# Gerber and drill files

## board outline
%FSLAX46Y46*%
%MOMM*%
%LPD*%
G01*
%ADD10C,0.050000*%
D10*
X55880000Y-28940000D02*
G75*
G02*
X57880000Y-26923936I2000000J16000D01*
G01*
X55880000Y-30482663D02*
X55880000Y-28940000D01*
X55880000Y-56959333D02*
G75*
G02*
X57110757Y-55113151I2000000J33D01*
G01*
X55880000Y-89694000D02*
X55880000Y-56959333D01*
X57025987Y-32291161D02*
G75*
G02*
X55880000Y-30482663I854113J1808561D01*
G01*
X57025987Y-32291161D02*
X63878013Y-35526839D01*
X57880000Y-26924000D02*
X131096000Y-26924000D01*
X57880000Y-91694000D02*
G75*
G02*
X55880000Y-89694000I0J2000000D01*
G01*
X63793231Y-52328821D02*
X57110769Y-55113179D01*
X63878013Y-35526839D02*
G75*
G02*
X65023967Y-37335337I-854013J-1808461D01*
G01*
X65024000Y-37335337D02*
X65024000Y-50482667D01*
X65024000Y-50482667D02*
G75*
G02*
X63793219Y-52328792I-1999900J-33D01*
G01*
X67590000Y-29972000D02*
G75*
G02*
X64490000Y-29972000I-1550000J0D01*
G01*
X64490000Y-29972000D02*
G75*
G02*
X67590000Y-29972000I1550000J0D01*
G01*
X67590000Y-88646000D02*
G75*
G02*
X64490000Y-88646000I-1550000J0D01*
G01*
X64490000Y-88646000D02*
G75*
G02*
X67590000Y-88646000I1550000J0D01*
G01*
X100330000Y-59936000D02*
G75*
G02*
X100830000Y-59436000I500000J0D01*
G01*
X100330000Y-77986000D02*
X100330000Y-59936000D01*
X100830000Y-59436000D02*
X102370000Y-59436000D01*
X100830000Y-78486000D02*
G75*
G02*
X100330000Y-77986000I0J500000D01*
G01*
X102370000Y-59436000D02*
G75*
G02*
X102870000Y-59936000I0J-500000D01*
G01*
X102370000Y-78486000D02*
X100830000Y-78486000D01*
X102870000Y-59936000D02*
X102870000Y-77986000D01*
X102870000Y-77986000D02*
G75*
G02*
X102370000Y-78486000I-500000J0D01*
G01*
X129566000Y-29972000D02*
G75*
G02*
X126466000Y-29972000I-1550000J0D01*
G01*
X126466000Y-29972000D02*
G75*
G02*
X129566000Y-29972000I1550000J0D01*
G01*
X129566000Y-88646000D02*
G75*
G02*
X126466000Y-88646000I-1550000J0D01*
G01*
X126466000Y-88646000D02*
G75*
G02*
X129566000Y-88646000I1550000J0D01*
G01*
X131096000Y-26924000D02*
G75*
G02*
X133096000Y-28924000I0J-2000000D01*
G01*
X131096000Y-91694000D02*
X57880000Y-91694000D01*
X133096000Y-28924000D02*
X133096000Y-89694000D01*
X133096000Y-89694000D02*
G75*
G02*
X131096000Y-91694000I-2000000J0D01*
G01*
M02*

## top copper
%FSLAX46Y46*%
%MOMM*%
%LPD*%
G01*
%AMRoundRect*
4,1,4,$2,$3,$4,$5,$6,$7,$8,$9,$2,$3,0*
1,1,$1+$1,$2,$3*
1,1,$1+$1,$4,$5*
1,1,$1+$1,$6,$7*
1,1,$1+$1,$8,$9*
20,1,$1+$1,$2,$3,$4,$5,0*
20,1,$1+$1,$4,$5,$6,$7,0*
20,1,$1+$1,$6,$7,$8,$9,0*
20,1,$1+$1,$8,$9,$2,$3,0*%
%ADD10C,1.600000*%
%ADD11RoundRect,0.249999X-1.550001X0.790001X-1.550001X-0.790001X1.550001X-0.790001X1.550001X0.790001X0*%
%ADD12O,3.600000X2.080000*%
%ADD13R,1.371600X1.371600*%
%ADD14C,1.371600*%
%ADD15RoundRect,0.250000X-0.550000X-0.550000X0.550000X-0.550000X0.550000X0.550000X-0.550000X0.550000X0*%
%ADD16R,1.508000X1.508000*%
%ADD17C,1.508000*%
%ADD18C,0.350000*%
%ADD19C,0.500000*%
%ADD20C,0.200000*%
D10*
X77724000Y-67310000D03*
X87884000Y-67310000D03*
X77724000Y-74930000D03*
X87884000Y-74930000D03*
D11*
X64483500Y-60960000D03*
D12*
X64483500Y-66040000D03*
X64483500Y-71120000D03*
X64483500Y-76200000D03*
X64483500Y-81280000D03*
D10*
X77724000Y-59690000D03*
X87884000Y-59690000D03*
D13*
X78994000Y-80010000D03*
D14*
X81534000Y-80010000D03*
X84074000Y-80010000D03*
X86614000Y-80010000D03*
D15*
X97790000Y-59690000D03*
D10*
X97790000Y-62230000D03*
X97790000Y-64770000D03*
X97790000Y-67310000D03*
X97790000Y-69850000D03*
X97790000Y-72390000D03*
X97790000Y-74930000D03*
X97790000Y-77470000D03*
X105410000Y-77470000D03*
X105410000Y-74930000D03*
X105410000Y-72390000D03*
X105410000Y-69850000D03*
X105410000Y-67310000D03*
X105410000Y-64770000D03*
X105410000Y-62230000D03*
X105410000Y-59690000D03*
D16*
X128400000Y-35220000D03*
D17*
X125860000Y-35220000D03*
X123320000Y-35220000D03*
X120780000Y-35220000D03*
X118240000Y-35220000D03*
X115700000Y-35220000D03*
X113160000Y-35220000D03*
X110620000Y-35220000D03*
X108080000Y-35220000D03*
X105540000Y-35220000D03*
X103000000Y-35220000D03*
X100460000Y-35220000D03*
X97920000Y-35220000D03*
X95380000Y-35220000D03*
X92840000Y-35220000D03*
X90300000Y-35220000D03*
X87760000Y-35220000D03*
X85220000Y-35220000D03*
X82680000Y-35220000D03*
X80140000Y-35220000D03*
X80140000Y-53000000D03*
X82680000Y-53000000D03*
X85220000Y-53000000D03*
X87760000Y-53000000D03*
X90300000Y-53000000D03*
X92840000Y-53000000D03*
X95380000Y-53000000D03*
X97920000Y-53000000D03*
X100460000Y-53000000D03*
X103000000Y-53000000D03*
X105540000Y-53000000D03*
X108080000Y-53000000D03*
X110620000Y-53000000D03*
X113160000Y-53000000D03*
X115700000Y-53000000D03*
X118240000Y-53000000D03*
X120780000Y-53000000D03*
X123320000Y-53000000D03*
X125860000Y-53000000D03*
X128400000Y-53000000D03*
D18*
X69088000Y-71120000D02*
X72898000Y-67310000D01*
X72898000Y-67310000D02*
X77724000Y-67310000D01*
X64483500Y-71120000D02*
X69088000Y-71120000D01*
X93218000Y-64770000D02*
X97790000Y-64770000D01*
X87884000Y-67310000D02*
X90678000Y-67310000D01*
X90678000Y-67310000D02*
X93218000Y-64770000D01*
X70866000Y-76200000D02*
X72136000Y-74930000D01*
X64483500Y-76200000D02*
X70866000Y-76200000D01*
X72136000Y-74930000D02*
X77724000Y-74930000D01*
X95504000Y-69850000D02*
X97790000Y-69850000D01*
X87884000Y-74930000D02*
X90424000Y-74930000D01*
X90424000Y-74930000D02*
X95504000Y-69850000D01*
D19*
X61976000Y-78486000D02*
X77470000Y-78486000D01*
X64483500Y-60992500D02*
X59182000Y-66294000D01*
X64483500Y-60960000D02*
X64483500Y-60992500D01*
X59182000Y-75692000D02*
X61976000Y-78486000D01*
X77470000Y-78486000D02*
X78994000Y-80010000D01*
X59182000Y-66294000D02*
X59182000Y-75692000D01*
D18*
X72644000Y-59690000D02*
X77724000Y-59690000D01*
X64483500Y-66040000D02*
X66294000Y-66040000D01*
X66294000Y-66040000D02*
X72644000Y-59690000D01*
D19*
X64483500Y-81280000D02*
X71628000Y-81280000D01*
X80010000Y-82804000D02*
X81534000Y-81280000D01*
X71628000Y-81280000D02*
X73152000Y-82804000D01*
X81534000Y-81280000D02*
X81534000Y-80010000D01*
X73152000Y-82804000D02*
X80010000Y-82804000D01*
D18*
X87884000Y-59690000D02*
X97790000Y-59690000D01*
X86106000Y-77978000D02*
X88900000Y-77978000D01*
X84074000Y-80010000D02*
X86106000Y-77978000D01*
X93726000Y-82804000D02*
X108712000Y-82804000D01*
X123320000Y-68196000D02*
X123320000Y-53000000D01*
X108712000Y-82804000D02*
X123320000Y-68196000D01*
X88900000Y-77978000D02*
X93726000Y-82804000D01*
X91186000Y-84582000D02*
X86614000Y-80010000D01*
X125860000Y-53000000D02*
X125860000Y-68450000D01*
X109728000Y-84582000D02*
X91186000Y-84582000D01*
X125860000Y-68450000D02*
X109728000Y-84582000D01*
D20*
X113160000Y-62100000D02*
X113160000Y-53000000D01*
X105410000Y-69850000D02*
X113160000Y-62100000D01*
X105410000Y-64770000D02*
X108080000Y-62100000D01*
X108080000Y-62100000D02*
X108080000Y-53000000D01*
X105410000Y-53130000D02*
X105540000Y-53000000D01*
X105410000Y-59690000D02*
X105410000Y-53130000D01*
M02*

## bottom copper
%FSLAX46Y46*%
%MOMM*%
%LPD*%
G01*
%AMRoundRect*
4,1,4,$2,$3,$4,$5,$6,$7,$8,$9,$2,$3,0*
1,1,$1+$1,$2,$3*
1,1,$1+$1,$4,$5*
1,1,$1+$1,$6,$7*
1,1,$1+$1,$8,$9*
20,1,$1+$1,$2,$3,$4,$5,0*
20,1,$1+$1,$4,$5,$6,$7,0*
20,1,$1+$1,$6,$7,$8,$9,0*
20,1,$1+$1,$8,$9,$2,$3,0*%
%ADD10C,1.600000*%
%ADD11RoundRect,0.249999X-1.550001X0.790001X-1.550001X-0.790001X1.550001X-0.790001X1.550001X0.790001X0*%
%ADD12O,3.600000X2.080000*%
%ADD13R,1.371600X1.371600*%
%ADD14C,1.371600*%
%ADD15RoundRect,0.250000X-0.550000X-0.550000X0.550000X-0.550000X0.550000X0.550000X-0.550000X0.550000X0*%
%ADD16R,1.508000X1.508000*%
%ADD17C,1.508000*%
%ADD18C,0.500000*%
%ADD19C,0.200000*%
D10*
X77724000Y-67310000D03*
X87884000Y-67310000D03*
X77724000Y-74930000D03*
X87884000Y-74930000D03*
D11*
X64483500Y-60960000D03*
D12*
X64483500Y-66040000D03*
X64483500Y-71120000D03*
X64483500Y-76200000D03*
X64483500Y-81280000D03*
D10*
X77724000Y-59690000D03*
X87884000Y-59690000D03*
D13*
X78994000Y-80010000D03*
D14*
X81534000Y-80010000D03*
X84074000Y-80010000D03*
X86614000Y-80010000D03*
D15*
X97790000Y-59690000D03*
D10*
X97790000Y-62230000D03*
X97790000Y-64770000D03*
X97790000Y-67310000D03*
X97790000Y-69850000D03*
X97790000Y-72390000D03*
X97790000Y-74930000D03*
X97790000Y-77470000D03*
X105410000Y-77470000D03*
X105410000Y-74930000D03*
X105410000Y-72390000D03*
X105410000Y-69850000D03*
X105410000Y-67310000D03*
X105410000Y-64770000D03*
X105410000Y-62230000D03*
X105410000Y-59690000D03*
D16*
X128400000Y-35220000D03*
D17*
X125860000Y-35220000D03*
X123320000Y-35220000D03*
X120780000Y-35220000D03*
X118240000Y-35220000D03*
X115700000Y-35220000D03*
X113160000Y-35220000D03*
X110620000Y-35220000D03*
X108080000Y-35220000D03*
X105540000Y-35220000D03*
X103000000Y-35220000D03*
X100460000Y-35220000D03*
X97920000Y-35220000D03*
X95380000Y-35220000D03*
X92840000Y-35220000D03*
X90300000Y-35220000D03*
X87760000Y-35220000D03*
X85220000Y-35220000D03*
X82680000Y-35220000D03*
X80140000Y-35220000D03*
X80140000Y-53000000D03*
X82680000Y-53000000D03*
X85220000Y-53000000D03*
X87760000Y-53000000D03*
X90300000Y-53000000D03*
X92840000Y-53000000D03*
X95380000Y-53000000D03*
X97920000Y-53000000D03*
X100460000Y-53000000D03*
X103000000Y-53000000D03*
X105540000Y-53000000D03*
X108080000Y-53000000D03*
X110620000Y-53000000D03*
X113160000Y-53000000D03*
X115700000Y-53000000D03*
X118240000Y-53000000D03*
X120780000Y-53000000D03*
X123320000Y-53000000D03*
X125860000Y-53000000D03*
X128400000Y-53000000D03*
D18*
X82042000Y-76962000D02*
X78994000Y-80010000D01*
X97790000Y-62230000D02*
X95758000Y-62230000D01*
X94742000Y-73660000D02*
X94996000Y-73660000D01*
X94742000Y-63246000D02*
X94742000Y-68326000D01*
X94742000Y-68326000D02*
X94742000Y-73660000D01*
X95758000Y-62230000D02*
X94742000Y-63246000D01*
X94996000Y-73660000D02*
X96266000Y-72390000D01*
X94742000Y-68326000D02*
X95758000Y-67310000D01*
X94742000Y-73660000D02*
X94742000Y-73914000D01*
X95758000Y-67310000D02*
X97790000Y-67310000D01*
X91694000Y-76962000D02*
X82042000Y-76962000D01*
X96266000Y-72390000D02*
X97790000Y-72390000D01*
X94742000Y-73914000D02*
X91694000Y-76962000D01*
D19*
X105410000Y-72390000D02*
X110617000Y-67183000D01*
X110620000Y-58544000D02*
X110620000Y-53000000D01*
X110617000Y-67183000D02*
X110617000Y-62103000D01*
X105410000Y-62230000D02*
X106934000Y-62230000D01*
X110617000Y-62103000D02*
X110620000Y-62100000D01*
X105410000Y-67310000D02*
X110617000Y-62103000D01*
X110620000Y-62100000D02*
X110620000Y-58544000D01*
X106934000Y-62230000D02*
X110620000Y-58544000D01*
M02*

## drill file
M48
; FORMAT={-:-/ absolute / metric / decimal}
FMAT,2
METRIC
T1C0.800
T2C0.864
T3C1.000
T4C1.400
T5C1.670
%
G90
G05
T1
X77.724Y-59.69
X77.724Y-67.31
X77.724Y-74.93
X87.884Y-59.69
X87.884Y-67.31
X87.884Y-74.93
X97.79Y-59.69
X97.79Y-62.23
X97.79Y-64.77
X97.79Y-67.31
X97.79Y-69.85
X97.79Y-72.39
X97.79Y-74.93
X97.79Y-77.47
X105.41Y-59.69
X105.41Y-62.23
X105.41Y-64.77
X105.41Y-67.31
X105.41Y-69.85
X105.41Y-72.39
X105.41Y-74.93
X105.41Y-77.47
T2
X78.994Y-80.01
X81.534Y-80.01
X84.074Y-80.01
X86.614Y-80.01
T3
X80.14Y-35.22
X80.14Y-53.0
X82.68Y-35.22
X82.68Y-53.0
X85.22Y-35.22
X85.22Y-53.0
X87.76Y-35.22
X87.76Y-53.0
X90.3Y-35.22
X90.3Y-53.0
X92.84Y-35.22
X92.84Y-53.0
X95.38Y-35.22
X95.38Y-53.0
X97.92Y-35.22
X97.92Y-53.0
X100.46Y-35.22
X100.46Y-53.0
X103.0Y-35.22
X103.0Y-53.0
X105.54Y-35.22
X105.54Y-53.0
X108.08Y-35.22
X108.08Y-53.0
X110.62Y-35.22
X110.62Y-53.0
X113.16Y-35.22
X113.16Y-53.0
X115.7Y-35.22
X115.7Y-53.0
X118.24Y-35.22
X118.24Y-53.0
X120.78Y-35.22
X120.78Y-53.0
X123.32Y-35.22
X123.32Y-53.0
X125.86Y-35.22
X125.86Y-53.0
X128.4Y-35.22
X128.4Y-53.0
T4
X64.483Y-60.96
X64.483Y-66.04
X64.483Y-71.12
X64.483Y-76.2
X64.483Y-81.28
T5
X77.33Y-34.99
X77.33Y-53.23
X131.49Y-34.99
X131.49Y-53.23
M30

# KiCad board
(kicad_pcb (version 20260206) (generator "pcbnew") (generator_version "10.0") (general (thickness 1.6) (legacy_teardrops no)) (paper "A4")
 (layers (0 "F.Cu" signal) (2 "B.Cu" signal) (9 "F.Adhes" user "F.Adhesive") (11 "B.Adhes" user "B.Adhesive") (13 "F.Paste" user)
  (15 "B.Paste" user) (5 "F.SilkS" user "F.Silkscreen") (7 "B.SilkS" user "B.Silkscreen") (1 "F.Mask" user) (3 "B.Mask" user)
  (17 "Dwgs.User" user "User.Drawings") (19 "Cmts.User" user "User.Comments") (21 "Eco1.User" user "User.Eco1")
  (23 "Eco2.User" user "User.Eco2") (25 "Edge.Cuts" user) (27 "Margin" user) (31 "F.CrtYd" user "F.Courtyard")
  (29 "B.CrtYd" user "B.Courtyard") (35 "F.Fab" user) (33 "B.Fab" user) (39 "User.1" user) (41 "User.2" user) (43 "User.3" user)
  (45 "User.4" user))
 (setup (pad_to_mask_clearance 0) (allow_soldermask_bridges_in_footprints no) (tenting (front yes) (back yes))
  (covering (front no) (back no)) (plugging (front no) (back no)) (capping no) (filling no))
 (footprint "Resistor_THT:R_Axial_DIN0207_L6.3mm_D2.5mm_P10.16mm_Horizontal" (layer "F.Cu") (at 77.724 67.31)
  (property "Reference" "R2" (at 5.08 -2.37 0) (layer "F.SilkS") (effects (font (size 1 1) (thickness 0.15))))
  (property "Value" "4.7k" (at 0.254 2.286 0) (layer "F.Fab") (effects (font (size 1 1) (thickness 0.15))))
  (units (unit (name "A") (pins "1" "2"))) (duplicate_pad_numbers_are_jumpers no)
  (pad "1" thru_hole circle (at 0 0) (size 1.6 1.6) (drill 0.8) (layers "*.Cu" "*.Mask") (remove_unused_layers no) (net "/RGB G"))
  (pad "2" thru_hole circle (at 10.16 0) (size 1.6 1.6) (drill 0.8) (layers "*.Cu" "*.Mask") (remove_unused_layers no) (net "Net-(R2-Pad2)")))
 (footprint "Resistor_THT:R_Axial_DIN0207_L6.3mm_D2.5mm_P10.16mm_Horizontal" (layer "F.Cu") (at 77.724 74.93)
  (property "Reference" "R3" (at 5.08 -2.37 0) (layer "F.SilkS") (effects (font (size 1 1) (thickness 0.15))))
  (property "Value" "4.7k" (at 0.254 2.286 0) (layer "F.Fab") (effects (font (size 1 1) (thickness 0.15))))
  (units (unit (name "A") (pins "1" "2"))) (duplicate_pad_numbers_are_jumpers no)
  (pad "1" thru_hole circle (at 0 0) (size 1.6 1.6) (drill 0.8) (layers "*.Cu" "*.Mask") (remove_unused_layers no) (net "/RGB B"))
  (pad "2" thru_hole circle (at 10.16 0) (size 1.6 1.6) (drill 0.8) (layers "*.Cu" "*.Mask") (remove_unused_layers no) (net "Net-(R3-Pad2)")))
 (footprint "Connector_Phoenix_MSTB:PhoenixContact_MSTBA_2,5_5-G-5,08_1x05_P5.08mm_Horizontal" (layer "F.Cu") (at 64.4835 60.96 -90)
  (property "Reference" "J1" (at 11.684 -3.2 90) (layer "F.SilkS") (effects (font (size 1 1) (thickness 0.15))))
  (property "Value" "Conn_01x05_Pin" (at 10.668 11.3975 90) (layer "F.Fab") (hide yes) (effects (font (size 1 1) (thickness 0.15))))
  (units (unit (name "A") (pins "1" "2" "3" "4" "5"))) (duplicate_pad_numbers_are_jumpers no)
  (pad "1" thru_hole roundrect (at 0 0 270) (size 2.08 3.6) (drill 1.4) (layers "*.Cu" "*.Mask") (remove_unused_layers no)
   (roundrect_rratio 0.120192) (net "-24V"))
  (pad "2" thru_hole oval (at 5.08 0 270) (size 2.08 3.6) (drill 1.4) (layers "*.Cu" "*.Mask") (remove_unused_layers no) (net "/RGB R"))
  (pad "3" thru_hole oval (at 10.16 0 270) (size 2.08 3.6) (drill 1.4) (layers "*.Cu" "*.Mask") (remove_unused_layers no) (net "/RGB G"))
  (pad "4" thru_hole oval (at 15.24 0 270) (size 2.08 3.6) (drill 1.4) (layers "*.Cu" "*.Mask") (remove_unused_layers no) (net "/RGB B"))
  (pad "5" thru_hole oval (at 20.32 0 270) (size 2.08 3.6) (drill 1.4) (layers "*.Cu" "*.Mask") (remove_unused_layers no) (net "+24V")))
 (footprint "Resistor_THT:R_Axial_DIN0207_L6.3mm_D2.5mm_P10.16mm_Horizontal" (layer "F.Cu") (at 77.724 59.69)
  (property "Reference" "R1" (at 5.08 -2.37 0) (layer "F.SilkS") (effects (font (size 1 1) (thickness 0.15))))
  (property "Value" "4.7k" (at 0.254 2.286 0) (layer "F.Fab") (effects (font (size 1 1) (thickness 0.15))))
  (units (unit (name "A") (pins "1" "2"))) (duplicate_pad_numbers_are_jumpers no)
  (pad "1" thru_hole circle (at 0 0) (size 1.6 1.6) (drill 0.8) (layers "*.Cu" "*.Mask") (remove_unused_layers no) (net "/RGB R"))
  (pad "2" thru_hole circle (at 10.16 0) (size 1.6 1.6) (drill 0.8) (layers "*.Cu" "*.Mask") (remove_unused_layers no) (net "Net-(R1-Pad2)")))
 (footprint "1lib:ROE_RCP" (layer "F.Cu") (at 78.994 80.01)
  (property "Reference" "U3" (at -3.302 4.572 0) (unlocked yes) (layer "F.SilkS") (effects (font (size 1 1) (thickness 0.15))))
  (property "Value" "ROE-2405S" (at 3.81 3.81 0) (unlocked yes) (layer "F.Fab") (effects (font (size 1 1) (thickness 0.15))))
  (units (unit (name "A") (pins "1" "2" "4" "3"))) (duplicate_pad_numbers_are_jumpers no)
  (pad "1" thru_hole rect (at 0 0) (size 1.3716 1.3716) (drill 0.8636) (layers "*.Cu" "*.Mask") (remove_unused_layers no) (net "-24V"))
  (pad "2" thru_hole circle (at 2.54 0) (size 1.3716 1.3716) (drill 0.8636) (layers "*.Cu" "*.Mask") (remove_unused_layers no) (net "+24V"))
  (pad "3" thru_hole circle (at 5.08 0) (size 1.3716 1.3716) (drill 0.8636) (layers "*.Cu" "*.Mask") (remove_unused_layers no) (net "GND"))
  (pad "4" thru_hole circle (at 7.62 0) (size 1.3716 1.3716) (drill 0.8636) (layers "*.Cu" "*.Mask") (remove_unused_layers no) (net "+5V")))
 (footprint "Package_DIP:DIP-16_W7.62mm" (layer "F.Cu") (at 97.79 59.69)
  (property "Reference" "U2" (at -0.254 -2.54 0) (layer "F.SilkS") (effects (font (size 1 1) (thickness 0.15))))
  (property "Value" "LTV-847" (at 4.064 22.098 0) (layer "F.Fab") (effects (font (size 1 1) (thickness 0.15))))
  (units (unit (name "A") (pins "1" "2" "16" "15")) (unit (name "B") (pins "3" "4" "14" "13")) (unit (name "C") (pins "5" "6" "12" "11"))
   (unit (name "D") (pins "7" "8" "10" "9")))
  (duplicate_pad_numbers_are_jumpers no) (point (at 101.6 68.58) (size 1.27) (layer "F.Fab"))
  (pad "1" thru_hole roundrect (at 0 0) (size 1.6 1.6) (drill 0.8) (layers "*.Cu" "*.Mask") (remove_unused_layers no)
   (roundrect_rratio 0.15625) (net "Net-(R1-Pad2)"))
  (pad "2" thru_hole circle (at 0 2.54) (size 1.6 1.6) (drill 0.8) (layers "*.Cu" "*.Mask") (remove_unused_layers no) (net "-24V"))
  (pad "3" thru_hole circle (at 0 5.08) (size 1.6 1.6) (drill 0.8) (layers "*.Cu" "*.Mask") (remove_unused_layers no) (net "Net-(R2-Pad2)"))
  (pad "4" thru_hole circle (at 0 7.62) (size 1.6 1.6) (drill 0.8) (layers "*.Cu" "*.Mask") (remove_unused_layers no) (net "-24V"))
  (pad "5" thru_hole circle (at 0 10.16) (size 1.6 1.6) (drill 0.8) (layers "*.Cu" "*.Mask") (remove_unused_layers no) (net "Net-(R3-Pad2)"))
  (pad "6" thru_hole circle (at 0 12.7) (size 1.6 1.6) (drill 0.8) (layers "*.Cu" "*.Mask") (remove_unused_layers no) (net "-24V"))
  (pad "7" thru_hole circle (at 0 15.24) (size 1.6 1.6) (drill 0.8) (layers "*.Cu" "*.Mask") (remove_unused_layers no))
  (pad "8" thru_hole circle (at 0 17.78) (size 1.6 1.6) (drill 0.8) (layers "*.Cu" "*.Mask") (remove_unused_layers no))
  (pad "9" thru_hole circle (at 7.62 17.78) (size 1.6 1.6) (drill 0.8) (layers "*.Cu" "*.Mask") (remove_unused_layers no))
  (pad "10" thru_hole circle (at 7.62 15.24) (size 1.6 1.6) (drill 0.8) (layers "*.Cu" "*.Mask") (remove_unused_layers no))
  (pad "11" thru_hole circle (at 7.62 12.7) (size 1.6 1.6) (drill 0.8) (layers "*.Cu" "*.Mask") (remove_unused_layers no) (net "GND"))
  (pad "12" thru_hole circle (at 7.62 10.16) (size 1.6 1.6) (drill 0.8) (layers "*.Cu" "*.Mask") (remove_unused_layers no)
   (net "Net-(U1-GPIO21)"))
  (pad "13" thru_hole circle (at 7.62 7.62) (size 1.6 1.6) (drill 0.8) (layers "*.Cu" "*.Mask") (remove_unused_layers no) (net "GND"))
  (pad "14" thru_hole circle (at 7.62 5.08) (size 1.6 1.6) (drill 0.8) (layers "*.Cu" "*.Mask") (remove_unused_layers no)
   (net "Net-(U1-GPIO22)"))
  (pad "15" thru_hole circle (at 7.62 2.54) (size 1.6 1.6) (drill 0.8) (layers "*.Cu" "*.Mask") (remove_unused_layers no) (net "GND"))
  (pad "16" thru_hole circle (at 7.62 0) (size 1.6 1.6) (drill 0.8) (layers "*.Cu" "*.Mask") (remove_unused_layers no)
   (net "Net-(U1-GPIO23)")))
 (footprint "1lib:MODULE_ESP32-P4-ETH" (layer "F.Cu") (at 94.07 44.11)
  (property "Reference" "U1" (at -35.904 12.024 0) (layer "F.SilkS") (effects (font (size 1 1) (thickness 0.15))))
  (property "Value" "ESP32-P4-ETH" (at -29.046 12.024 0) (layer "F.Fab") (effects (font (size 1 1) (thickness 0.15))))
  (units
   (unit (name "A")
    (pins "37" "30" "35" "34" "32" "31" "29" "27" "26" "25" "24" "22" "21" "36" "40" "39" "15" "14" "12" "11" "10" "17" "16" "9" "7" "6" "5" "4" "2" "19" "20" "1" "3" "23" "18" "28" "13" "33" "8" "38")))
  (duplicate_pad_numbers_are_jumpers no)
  (pad "" np_thru_hole circle (at -16.74 -9.12) (size 1.67 1.67) (drill 1.67) (layers "*.Cu" "*.Mask"))
  (pad "" np_thru_hole circle (at -16.74 9.12) (size 1.67 1.67) (drill 1.67) (layers "*.Cu" "*.Mask"))
  (pad "" np_thru_hole circle (at 37.42 -9.12) (size 1.67 1.67) (drill 1.67) (layers "*.Cu" "*.Mask"))
  (pad "" np_thru_hole circle (at 37.42 9.12) (size 1.67 1.67) (drill 1.67) (layers "*.Cu" "*.Mask"))
  (pad "1" thru_hole rect (at 34.33 -8.89) (size 1.508 1.508) (drill 1) (layers "*.Cu" "*.Mask") (remove_unused_layers no)
   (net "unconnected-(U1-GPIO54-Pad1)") (solder_mask_margin 0.102))
  (pad "2" thru_hole circle (at 31.79 -8.89) (size 1.508 1.508) (drill 1) (layers "*.Cu" "*.Mask") (remove_unused_layers no)
   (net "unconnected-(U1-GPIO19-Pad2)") (solder_mask_margin 0.102))
  (pad "3" thru_hole circle (at 29.25 -8.89) (size 1.508 1.508) (drill 1) (layers "*.Cu" "*.Mask") (remove_unused_layers no) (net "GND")
   (solder_mask_margin 0.102))
  (pad "4" thru_hole circle (at 26.71 -8.89) (size 1.508 1.508) (drill 1) (layers "*.Cu" "*.Mask") (remove_unused_layers no)
   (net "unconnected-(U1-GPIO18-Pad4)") (solder_mask_margin 0.102))
  (pad "5" thru_hole circle (at 24.17 -8.89) (size 1.508 1.508) (drill 1) (layers "*.Cu" "*.Mask") (remove_unused_layers no)
   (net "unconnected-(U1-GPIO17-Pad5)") (solder_mask_margin 0.102))
  (pad "6" thru_hole circle (at 21.63 -8.89) (size 1.508 1.508) (drill 1) (layers "*.Cu" "*.Mask") (remove_unused_layers no)
   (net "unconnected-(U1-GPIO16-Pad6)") (solder_mask_margin 0.102))
  (pad "7" thru_hole circle (at 19.09 -8.89) (size 1.508 1.508) (drill 1) (layers "*.Cu" "*.Mask") (remove_unused_layers no)
   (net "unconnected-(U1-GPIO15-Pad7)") (solder_mask_margin 0.102))
  (pad "8" thru_hole circle (at 16.55 -8.89) (size 1.508 1.508) (drill 1) (layers "*.Cu" "*.Mask") (remove_unused_layers no) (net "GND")
   (solder_mask_margin 0.102))
  (pad "9" thru_hole circle (at 14.01 -8.89) (size 1.508 1.508) (drill 1) (layers "*.Cu" "*.Mask") (remove_unused_layers no)
   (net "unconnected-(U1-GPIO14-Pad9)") (solder_mask_margin 0.102))
  (pad "10" thru_hole circle (at 11.47 -8.89) (size 1.508 1.508) (drill 1) (layers "*.Cu" "*.Mask") (remove_unused_layers no)
   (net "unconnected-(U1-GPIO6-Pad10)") (solder_mask_margin 0.102))
  (pad "11" thru_hole circle (at 8.93 -8.89) (size 1.508 1.508) (drill 1) (layers "*.Cu" "*.Mask") (remove_unused_layers no)
   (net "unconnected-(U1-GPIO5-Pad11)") (solder_mask_margin 0.102))
  (pad "12" thru_hole circle (at 6.39 -8.89) (size 1.508 1.508) (drill 1) (layers "*.Cu" "*.Mask") (remove_unused_layers no)
   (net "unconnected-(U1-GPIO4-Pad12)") (solder_mask_margin 0.102))
  (pad "13" thru_hole circle (at 3.85 -8.89) (size 1.508 1.508) (drill 1) (layers "*.Cu" "*.Mask") (remove_unused_layers no) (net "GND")
   (solder_mask_margin 0.102))
  (pad "14" thru_hole circle (at 1.31 -8.89) (size 1.508 1.508) (drill 1) (layers "*.Cu" "*.Mask") (remove_unused_layers no)
   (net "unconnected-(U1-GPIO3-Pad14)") (solder_mask_margin 0.102))
  (pad "15" thru_hole circle (at -1.23 -8.89) (size 1.508 1.508) (drill 1) (layers "*.Cu" "*.Mask") (remove_unused_layers no)
   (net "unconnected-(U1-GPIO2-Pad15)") (solder_mask_margin 0.102))
  (pad "16" thru_hole circle (at -3.77 -8.89) (size 1.508 1.508) (drill 1) (layers "*.Cu" "*.Mask") (remove_unused_layers no)
   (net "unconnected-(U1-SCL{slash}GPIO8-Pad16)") (solder_mask_margin 0.102))
  (pad "17" thru_hole circle (at -6.31 -8.89) (size 1.508 1.508) (drill 1) (layers "*.Cu" "*.Mask") (remove_unused_layers no)
   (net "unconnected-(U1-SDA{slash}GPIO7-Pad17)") (solder_mask_margin 0.102))
  (pad "18" thru_hole circle (at -8.85 -8.89) (size 1.508 1.508) (drill 1) (layers "*.Cu" "*.Mask") (remove_unused_layers no) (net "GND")
   (solder_mask_margin 0.102))
  (pad "19" thru_hole circle (at -11.39 -8.89) (size 1.508 1.508) (drill 1) (layers "*.Cu" "*.Mask") (remove_unused_layers no)
   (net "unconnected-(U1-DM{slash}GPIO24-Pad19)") (solder_mask_margin 0.102))
  (pad "20" thru_hole circle (at -13.93 -8.89) (size 1.508 1.508) (drill 1) (layers "*.Cu" "*.Mask") (remove_unused_layers no)
   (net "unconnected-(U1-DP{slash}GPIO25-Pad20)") (solder_mask_margin 0.102))
  (pad "21" thru_hole circle (at -13.93 8.89) (size 1.508 1.508) (drill 1) (layers "*.Cu" "*.Mask") (remove_unused_layers no)
   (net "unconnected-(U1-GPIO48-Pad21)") (solder_mask_margin 0.102))
  (pad "22" thru_hole circle (at -11.39 8.89) (size 1.508 1.508) (drill 1) (layers "*.Cu" "*.Mask") (remove_unused_layers no)
   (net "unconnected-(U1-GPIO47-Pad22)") (solder_mask_margin 0.102))
  (pad "23" thru_hole circle (at -8.85 8.89) (size 1.508 1.508) (drill 1) (layers "*.Cu" "*.Mask") (remove_unused_layers no) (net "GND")
   (solder_mask_margin 0.102))
  (pad "24" thru_hole circle (at -6.31 8.89) (size 1.508 1.508) (drill 1) (layers "*.Cu" "*.Mask") (remove_unused_layers no)
   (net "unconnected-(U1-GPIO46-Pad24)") (solder_mask_margin 0.102))
  (pad "25" thru_hole circle (at -3.77 8.89) (size 1.508 1.508) (drill 1) (layers "*.Cu" "*.Mask") (remove_unused_layers no)
   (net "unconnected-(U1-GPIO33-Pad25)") (solder_mask_margin 0.102))
  (pad "26" thru_hole circle (at -1.23 8.89) (size 1.508 1.508) (drill 1) (layers "*.Cu" "*.Mask") (remove_unused_layers no)
   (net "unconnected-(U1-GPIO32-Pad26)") (solder_mask_margin 0.102))
  (pad "27" thru_hole circle (at 1.31 8.89) (size 1.508 1.508) (drill 1) (layers "*.Cu" "*.Mask") (remove_unused_layers no)
   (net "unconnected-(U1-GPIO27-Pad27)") (solder_mask_margin 0.102))
  (pad "28" thru_hole circle (at 3.85 8.89) (size 1.508 1.508) (drill 1) (layers "*.Cu" "*.Mask") (remove_unused_layers no) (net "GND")
   (solder_mask_margin 0.102))
  (pad "29" thru_hole circle (at 6.39 8.89) (size 1.508 1.508) (drill 1) (layers "*.Cu" "*.Mask") (remove_unused_layers no)
   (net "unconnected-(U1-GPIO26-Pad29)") (solder_mask_margin 0.102))
  (pad "30" thru_hole circle (at 8.93 8.89) (size 1.508 1.508) (drill 1) (layers "*.Cu" "*.Mask") (remove_unused_layers no)
   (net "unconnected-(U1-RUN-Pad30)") (solder_mask_margin 0.102))
  (pad "31" thru_hole circle (at 11.47 8.89) (size 1.508 1.508) (drill 1) (layers "*.Cu" "*.Mask") (remove_unused_layers no)
   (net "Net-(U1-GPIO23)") (solder_mask_margin 0.102))
  (pad "32" thru_hole circle (at 14.01 8.89) (size 1.508 1.508) (drill 1) (layers "*.Cu" "*.Mask") (remove_unused_layers no)
   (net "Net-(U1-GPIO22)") (solder_mask_margin 0.102))
  (pad "33" thru_hole circle (at 16.55 8.89) (size 1.508 1.508) (drill 1) (layers "*.Cu" "*.Mask") (remove_unused_layers no) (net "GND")
   (solder_mask_margin 0.102))
  (pad "34" thru_hole circle (at 19.09 8.89) (size 1.508 1.508) (drill 1) (layers "*.Cu" "*.Mask") (remove_unused_layers no)
   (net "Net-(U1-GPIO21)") (solder_mask_margin 0.102))
  (pad "35" thru_hole circle (at 21.63 8.89) (size 1.508 1.508) (drill 1) (layers "*.Cu" "*.Mask") (remove_unused_layers no)
   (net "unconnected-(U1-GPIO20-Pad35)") (solder_mask_margin 0.102))
  (pad "36" thru_hole circle (at 24.17 8.89) (size 1.508 1.508) (drill 1) (layers "*.Cu" "*.Mask") (remove_unused_layers no)
   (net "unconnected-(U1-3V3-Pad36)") (solder_mask_margin 0.102))
  (pad "37" thru_hole circle (at 26.71 8.89) (size 1.508 1.508) (drill 1) (layers "*.Cu" "*.Mask") (remove_unused_layers no)
   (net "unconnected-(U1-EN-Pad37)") (solder_mask_margin 0.102))
  (pad "38" thru_hole circle (at 29.25 8.89) (size 1.508 1.508) (drill 1) (layers "*.Cu" "*.Mask") (remove_unused_layers no) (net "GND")
   (solder_mask_margin 0.102))
  (pad "39" thru_hole circle (at 31.79 8.89) (size 1.508 1.508) (drill 1) (layers "*.Cu" "*.Mask") (remove_unused_layers no) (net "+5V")
   (solder_mask_margin 0.102))
  (pad "40" thru_hole circle (at 34.33 8.89) (size 1.508 1.508) (drill 1) (layers "*.Cu" "*.Mask") (remove_unused_layers no)
   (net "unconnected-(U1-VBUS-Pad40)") (solder_mask_margin 0.102)))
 (gr_arc (start 55.88 28.94) (mid 56.460096 27.515409) (end 57.88 26.923936) (stroke (width 0.05) (type default)) (layer "Edge.Cuts"))
 (gr_line (start 55.88 30.482663) (end 55.88 28.94) (stroke (width 0.05) (type default)) (layer "Edge.Cuts"))
 (gr_arc (start 55.88 56.959333) (mid 56.215899 55.849933) (end 57.110769 55.113179) (stroke (width 0.05) (type default))
  (layer "Edge.Cuts"))
 (gr_line (start 55.88 89.694) (end 55.88 56.959333) (stroke (width 0.05) (type default)) (layer "Edge.Cuts"))
 (gr_arc (start 57.025987 32.291161) (mid 56.190631 31.553168) (end 55.88 30.482663) (stroke (width 0.05) (type default))
  (layer "Edge.Cuts"))
 (gr_line (start 57.025987 32.291161) (end 63.878013 35.526839) (stroke (width 0.05) (type default)) (layer "Edge.Cuts"))
 (gr_line (start 57.88 26.924) (end 131.096 26.924) (stroke (width 0.05) (type default)) (layer "Edge.Cuts"))
 (gr_arc (start 57.88 91.694) (mid 56.465786 91.108214) (end 55.88 89.694) (stroke (width 0.05) (type default)) (layer "Edge.Cuts"))
 (gr_line (start 63.793231 52.328821) (end 57.110769 55.113179) (stroke (width 0.05) (type default)) (layer "Edge.Cuts"))
 (gr_arc (start 63.878013 35.526839) (mid 64.713383 36.264829) (end 65.024 37.335337) (stroke (width 0.05) (type default))
  (layer "Edge.Cuts"))
 (gr_line (start 65.024 37.335337) (end 65.024 50.482667) (stroke (width 0.05) (type default)) (layer "Edge.Cuts"))
 (gr_arc (start 65.024 50.482667) (mid 64.688113 51.592081) (end 63.793231 52.328821) (stroke (width 0.05) (type default))
  (layer "Edge.Cuts"))
 (gr_circle (center 66.04 29.972) (end 67.59 29.972) (stroke (width 0.05) (type solid)) (fill no) (layer "Edge.Cuts"))
 (gr_circle (center 66.04 88.646) (end 67.59 88.646) (stroke (width 0.05) (type solid)) (fill no) (layer "Edge.Cuts"))
 (gr_arc (start 100.33 59.936) (mid 100.476447 59.582447) (end 100.83 59.436) (stroke (width 0.05) (type default)) (layer "Edge.Cuts"))
 (gr_line (start 100.33 77.986) (end 100.33 59.936) (stroke (width 0.05) (type default)) (layer "Edge.Cuts"))
 (gr_line (start 100.83 59.436) (end 102.37 59.436) (stroke (width 0.05) (type default)) (layer "Edge.Cuts"))
 (gr_arc (start 100.83 78.486) (mid 100.476447 78.339553) (end 100.33 77.986) (stroke (width 0.05) (type default)) (layer "Edge.Cuts"))
 (gr_arc (start 102.37 59.436) (mid 102.723553 59.582447) (end 102.87 59.936) (stroke (width 0.05) (type default)) (layer "Edge.Cuts"))
 (gr_line (start 102.37 78.486) (end 100.83 78.486) (stroke (width 0.05) (type default)) (layer "Edge.Cuts"))
 (gr_line (start 102.87 59.936) (end 102.87 77.986) (stroke (width 0.05) (type default)) (layer "Edge.Cuts"))
 (gr_arc (start 102.87 77.986) (mid 102.723553 78.339553) (end 102.37 78.486) (stroke (width 0.05) (type default)) (layer "Edge.Cuts"))
 (gr_circle (center 128.016 29.972) (end 129.566 29.972) (stroke (width 0.05) (type solid)) (fill no) (layer "Edge.Cuts"))
 (gr_circle (center 128.016 88.646) (end 129.566 88.646) (stroke (width 0.05) (type solid)) (fill no) (layer "Edge.Cuts"))
 (gr_arc (start 131.096 26.924) (mid 132.510214 27.509786) (end 133.096 28.924) (stroke (width 0.05) (type default)) (layer "Edge.Cuts"))
 (gr_line (start 131.096 91.694) (end 57.88 91.694) (stroke (width 0.05) (type default)) (layer "Edge.Cuts"))
 (gr_line (start 133.096 28.924) (end 133.096 89.694) (stroke (width 0.05) (type default)) (layer "Edge.Cuts"))
 (gr_arc (start 133.096 89.694) (mid 132.510214 91.108214) (end 131.096 91.694) (stroke (width 0.05) (type default)) (layer "Edge.Cuts"))
 (segment (start 69.088 71.12) (end 72.898 67.31) (width 0.35) (layer "F.Cu") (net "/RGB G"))
 (segment (start 72.898 67.31) (end 77.724 67.31) (width 0.35) (layer "F.Cu") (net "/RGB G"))
 (segment (start 64.4835 71.12) (end 69.088 71.12) (width 0.35) (layer "F.Cu") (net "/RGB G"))
 (segment (start 93.218 64.77) (end 97.79 64.77) (width 0.35) (layer "F.Cu") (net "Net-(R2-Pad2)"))
 (segment (start 87.884 67.31) (end 90.678 67.31) (width 0.35) (layer "F.Cu") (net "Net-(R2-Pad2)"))
 (segment (start 90.678 67.31) (end 93.218 64.77) (width 0.35) (layer "F.Cu") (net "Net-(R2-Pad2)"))
 (segment (start 70.866 76.2) (end 72.136 74.93) (width 0.35) (layer "F.Cu") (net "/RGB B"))
 (segment (start 64.4835 76.2) (end 70.866 76.2) (width 0.35) (layer "F.Cu") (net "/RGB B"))
 (segment (start 72.136 74.93) (end 77.724 74.93) (width 0.35) (layer "F.Cu") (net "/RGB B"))
 (segment (start 95.504 69.85) (end 97.79 69.85) (width 0.35) (layer "F.Cu") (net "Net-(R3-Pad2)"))
 (segment (start 87.884 74.93) (end 90.424 74.93) (width 0.35) (layer "F.Cu") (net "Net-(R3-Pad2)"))
 (segment (start 90.424 74.93) (end 95.504 69.85) (width 0.35) (layer "F.Cu") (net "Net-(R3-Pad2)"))
 (segment (start 61.976 78.486) (end 77.47 78.486) (width 0.5) (layer "F.Cu") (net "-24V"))
 (segment (start 64.4835 60.9925) (end 59.182 66.294) (width 0.5) (layer "F.Cu") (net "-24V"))
 (segment (start 64.4835 60.96) (end 64.4835 60.9925) (width 0.5) (layer "F.Cu") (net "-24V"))
 (segment (start 59.182 75.692) (end 61.976 78.486) (width 0.5) (layer "F.Cu") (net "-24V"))
 (segment (start 77.47 78.486) (end 78.994 80.01) (width 0.5) (layer "F.Cu") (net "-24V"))
 (segment (start 59.182 66.294) (end 59.182 75.692) (width 0.5) (layer "F.Cu") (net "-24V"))
 (segment (start 82.042 76.962) (end 78.994 80.01) (width 0.5) (layer "B.Cu") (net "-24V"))
 (segment (start 97.79 62.23) (end 95.758 62.23) (width 0.5) (layer "B.Cu") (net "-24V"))
 (segment (start 94.742 73.66) (end 94.996 73.66) (width 0.5) (layer "B.Cu") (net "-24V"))
 (segment (start 94.742 63.246) (end 94.742 68.326) (width 0.5) (layer "B.Cu") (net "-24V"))
 (segment (start 94.742 68.326) (end 94.742 73.66) (width 0.5) (layer "B.Cu") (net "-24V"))
 (segment (start 95.758 62.23) (end 94.742 63.246) (width 0.5) (layer "B.Cu") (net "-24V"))
 (segment (start 94.996 73.66) (end 96.266 72.39) (width 0.5) (layer "B.Cu") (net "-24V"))
 (segment (start 94.742 68.326) (end 95.758 67.31) (width 0.5) (layer "B.Cu") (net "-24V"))
 (segment (start 94.742 73.66) (end 94.742 73.914) (width 0.5) (layer "B.Cu") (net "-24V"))
 (segment (start 95.758 67.31) (end 97.79 67.31) (width 0.5) (layer "B.Cu") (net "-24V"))
 (segment (start 91.694 76.962) (end 82.042 76.962) (width 0.5) (layer "B.Cu") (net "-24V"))
 (segment (start 96.266 72.39) (end 97.79 72.39) (width 0.5) (layer "B.Cu") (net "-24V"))
 (segment (start 94.742 73.914) (end 91.694 76.962) (width 0.5) (layer "B.Cu") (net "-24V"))
 (segment (start 72.644 59.69) (end 77.724 59.69) (width 0.35) (layer "F.Cu") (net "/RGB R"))
 (segment (start 64.4835 66.04) (end 66.294 66.04) (width 0.35) (layer "F.Cu") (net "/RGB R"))
 (segment (start 66.294 66.04) (end 72.644 59.69) (width 0.35) (layer "F.Cu") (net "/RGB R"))
 (segment (start 64.4835 81.28) (end 71.628 81.28) (width 0.5) (layer "F.Cu") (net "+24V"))
 (segment (start 80.01 82.804) (end 81.534 81.28) (width 0.5) (layer "F.Cu") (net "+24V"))
 (segment (start 71.628 81.28) (end 73.152 82.804) (width 0.5) (layer "F.Cu") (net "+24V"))
 (segment (start 81.534 81.28) (end 81.534 80.01) (width 0.5) (layer "F.Cu") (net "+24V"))
 (segment (start 73.152 82.804) (end 80.01 82.804) (width 0.5) (layer "F.Cu") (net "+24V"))
 (segment (start 87.884 59.69) (end 97.79 59.69) (width 0.35) (layer "F.Cu") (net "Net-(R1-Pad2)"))
 (segment (start 86.106 77.978) (end 88.9 77.978) (width 0.35) (layer "F.Cu") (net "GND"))
 (segment (start 84.074 80.01) (end 86.106 77.978) (width 0.35) (layer "F.Cu") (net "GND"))
 (segment (start 93.726 82.804) (end 108.712 82.804) (width 0.35) (layer "F.Cu") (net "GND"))
 (segment (start 123.32 68.196) (end 123.32 53) (width 0.35) (layer "F.Cu") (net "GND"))
 (segment (start 108.712 82.804) (end 123.32 68.196) (width 0.35) (layer "F.Cu") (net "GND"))
 (segment (start 88.9 77.978) (end 93.726 82.804) (width 0.35) (layer "F.Cu") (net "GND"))
 (segment (start 105.41 72.39) (end 110.617 67.183) (width 0.2) (layer "B.Cu") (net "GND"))
 (segment (start 110.62 58.544) (end 110.62 53) (width 0.2) (layer "B.Cu") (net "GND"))
 (segment (start 110.617 67.183) (end 110.617 62.103) (width 0.2) (layer "B.Cu") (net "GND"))
 (segment (start 105.41 62.23) (end 106.934 62.23) (width 0.2) (layer "B.Cu") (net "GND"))
 (segment (start 110.617 62.103) (end 110.62 62.1) (width 0.2) (layer "B.Cu") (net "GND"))
 (segment (start 105.41 67.31) (end 110.617 62.103) (width 0.2) (layer "B.Cu") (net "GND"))
 (segment (start 110.62 62.1) (end 110.62 58.544) (width 0.2) (layer "B.Cu") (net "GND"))
 (segment (start 106.934 62.23) (end 110.62 58.544) (width 0.2) (layer "B.Cu") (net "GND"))
 (segment (start 91.186 84.582) (end 86.614 80.01) (width 0.35) (layer "F.Cu") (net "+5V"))
 (segment (start 125.86 53) (end 125.86 68.45) (width 0.35) (layer "F.Cu") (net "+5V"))
 (segment (start 109.728 84.582) (end 91.186 84.582) (width 0.35) (layer "F.Cu") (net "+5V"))
 (segment (start 125.86 68.45) (end 109.728 84.582) (width 0.35) (layer "F.Cu") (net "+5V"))
 (segment (start 113.16 62.1) (end 113.16 53) (width 0.2) (layer "F.Cu") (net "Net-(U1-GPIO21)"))
 (segment (start 105.41 69.85) (end 113.16 62.1) (width 0.2) (layer "F.Cu") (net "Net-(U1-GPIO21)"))
 (segment (start 105.41 64.77) (end 108.08 62.1) (width 0.2) (layer "F.Cu") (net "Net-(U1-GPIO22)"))
 (segment (start 108.08 62.1) (end 108.08 53) (width 0.2) (layer "F.Cu") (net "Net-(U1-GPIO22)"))
 (segment (start 105.41 53.13) (end 105.54 53) (width 0.2) (layer "F.Cu") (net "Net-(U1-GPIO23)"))
 (segment (start 105.41 59.69) (end 105.41 53.13) (width 0.2) (layer "F.Cu") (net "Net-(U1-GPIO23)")))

